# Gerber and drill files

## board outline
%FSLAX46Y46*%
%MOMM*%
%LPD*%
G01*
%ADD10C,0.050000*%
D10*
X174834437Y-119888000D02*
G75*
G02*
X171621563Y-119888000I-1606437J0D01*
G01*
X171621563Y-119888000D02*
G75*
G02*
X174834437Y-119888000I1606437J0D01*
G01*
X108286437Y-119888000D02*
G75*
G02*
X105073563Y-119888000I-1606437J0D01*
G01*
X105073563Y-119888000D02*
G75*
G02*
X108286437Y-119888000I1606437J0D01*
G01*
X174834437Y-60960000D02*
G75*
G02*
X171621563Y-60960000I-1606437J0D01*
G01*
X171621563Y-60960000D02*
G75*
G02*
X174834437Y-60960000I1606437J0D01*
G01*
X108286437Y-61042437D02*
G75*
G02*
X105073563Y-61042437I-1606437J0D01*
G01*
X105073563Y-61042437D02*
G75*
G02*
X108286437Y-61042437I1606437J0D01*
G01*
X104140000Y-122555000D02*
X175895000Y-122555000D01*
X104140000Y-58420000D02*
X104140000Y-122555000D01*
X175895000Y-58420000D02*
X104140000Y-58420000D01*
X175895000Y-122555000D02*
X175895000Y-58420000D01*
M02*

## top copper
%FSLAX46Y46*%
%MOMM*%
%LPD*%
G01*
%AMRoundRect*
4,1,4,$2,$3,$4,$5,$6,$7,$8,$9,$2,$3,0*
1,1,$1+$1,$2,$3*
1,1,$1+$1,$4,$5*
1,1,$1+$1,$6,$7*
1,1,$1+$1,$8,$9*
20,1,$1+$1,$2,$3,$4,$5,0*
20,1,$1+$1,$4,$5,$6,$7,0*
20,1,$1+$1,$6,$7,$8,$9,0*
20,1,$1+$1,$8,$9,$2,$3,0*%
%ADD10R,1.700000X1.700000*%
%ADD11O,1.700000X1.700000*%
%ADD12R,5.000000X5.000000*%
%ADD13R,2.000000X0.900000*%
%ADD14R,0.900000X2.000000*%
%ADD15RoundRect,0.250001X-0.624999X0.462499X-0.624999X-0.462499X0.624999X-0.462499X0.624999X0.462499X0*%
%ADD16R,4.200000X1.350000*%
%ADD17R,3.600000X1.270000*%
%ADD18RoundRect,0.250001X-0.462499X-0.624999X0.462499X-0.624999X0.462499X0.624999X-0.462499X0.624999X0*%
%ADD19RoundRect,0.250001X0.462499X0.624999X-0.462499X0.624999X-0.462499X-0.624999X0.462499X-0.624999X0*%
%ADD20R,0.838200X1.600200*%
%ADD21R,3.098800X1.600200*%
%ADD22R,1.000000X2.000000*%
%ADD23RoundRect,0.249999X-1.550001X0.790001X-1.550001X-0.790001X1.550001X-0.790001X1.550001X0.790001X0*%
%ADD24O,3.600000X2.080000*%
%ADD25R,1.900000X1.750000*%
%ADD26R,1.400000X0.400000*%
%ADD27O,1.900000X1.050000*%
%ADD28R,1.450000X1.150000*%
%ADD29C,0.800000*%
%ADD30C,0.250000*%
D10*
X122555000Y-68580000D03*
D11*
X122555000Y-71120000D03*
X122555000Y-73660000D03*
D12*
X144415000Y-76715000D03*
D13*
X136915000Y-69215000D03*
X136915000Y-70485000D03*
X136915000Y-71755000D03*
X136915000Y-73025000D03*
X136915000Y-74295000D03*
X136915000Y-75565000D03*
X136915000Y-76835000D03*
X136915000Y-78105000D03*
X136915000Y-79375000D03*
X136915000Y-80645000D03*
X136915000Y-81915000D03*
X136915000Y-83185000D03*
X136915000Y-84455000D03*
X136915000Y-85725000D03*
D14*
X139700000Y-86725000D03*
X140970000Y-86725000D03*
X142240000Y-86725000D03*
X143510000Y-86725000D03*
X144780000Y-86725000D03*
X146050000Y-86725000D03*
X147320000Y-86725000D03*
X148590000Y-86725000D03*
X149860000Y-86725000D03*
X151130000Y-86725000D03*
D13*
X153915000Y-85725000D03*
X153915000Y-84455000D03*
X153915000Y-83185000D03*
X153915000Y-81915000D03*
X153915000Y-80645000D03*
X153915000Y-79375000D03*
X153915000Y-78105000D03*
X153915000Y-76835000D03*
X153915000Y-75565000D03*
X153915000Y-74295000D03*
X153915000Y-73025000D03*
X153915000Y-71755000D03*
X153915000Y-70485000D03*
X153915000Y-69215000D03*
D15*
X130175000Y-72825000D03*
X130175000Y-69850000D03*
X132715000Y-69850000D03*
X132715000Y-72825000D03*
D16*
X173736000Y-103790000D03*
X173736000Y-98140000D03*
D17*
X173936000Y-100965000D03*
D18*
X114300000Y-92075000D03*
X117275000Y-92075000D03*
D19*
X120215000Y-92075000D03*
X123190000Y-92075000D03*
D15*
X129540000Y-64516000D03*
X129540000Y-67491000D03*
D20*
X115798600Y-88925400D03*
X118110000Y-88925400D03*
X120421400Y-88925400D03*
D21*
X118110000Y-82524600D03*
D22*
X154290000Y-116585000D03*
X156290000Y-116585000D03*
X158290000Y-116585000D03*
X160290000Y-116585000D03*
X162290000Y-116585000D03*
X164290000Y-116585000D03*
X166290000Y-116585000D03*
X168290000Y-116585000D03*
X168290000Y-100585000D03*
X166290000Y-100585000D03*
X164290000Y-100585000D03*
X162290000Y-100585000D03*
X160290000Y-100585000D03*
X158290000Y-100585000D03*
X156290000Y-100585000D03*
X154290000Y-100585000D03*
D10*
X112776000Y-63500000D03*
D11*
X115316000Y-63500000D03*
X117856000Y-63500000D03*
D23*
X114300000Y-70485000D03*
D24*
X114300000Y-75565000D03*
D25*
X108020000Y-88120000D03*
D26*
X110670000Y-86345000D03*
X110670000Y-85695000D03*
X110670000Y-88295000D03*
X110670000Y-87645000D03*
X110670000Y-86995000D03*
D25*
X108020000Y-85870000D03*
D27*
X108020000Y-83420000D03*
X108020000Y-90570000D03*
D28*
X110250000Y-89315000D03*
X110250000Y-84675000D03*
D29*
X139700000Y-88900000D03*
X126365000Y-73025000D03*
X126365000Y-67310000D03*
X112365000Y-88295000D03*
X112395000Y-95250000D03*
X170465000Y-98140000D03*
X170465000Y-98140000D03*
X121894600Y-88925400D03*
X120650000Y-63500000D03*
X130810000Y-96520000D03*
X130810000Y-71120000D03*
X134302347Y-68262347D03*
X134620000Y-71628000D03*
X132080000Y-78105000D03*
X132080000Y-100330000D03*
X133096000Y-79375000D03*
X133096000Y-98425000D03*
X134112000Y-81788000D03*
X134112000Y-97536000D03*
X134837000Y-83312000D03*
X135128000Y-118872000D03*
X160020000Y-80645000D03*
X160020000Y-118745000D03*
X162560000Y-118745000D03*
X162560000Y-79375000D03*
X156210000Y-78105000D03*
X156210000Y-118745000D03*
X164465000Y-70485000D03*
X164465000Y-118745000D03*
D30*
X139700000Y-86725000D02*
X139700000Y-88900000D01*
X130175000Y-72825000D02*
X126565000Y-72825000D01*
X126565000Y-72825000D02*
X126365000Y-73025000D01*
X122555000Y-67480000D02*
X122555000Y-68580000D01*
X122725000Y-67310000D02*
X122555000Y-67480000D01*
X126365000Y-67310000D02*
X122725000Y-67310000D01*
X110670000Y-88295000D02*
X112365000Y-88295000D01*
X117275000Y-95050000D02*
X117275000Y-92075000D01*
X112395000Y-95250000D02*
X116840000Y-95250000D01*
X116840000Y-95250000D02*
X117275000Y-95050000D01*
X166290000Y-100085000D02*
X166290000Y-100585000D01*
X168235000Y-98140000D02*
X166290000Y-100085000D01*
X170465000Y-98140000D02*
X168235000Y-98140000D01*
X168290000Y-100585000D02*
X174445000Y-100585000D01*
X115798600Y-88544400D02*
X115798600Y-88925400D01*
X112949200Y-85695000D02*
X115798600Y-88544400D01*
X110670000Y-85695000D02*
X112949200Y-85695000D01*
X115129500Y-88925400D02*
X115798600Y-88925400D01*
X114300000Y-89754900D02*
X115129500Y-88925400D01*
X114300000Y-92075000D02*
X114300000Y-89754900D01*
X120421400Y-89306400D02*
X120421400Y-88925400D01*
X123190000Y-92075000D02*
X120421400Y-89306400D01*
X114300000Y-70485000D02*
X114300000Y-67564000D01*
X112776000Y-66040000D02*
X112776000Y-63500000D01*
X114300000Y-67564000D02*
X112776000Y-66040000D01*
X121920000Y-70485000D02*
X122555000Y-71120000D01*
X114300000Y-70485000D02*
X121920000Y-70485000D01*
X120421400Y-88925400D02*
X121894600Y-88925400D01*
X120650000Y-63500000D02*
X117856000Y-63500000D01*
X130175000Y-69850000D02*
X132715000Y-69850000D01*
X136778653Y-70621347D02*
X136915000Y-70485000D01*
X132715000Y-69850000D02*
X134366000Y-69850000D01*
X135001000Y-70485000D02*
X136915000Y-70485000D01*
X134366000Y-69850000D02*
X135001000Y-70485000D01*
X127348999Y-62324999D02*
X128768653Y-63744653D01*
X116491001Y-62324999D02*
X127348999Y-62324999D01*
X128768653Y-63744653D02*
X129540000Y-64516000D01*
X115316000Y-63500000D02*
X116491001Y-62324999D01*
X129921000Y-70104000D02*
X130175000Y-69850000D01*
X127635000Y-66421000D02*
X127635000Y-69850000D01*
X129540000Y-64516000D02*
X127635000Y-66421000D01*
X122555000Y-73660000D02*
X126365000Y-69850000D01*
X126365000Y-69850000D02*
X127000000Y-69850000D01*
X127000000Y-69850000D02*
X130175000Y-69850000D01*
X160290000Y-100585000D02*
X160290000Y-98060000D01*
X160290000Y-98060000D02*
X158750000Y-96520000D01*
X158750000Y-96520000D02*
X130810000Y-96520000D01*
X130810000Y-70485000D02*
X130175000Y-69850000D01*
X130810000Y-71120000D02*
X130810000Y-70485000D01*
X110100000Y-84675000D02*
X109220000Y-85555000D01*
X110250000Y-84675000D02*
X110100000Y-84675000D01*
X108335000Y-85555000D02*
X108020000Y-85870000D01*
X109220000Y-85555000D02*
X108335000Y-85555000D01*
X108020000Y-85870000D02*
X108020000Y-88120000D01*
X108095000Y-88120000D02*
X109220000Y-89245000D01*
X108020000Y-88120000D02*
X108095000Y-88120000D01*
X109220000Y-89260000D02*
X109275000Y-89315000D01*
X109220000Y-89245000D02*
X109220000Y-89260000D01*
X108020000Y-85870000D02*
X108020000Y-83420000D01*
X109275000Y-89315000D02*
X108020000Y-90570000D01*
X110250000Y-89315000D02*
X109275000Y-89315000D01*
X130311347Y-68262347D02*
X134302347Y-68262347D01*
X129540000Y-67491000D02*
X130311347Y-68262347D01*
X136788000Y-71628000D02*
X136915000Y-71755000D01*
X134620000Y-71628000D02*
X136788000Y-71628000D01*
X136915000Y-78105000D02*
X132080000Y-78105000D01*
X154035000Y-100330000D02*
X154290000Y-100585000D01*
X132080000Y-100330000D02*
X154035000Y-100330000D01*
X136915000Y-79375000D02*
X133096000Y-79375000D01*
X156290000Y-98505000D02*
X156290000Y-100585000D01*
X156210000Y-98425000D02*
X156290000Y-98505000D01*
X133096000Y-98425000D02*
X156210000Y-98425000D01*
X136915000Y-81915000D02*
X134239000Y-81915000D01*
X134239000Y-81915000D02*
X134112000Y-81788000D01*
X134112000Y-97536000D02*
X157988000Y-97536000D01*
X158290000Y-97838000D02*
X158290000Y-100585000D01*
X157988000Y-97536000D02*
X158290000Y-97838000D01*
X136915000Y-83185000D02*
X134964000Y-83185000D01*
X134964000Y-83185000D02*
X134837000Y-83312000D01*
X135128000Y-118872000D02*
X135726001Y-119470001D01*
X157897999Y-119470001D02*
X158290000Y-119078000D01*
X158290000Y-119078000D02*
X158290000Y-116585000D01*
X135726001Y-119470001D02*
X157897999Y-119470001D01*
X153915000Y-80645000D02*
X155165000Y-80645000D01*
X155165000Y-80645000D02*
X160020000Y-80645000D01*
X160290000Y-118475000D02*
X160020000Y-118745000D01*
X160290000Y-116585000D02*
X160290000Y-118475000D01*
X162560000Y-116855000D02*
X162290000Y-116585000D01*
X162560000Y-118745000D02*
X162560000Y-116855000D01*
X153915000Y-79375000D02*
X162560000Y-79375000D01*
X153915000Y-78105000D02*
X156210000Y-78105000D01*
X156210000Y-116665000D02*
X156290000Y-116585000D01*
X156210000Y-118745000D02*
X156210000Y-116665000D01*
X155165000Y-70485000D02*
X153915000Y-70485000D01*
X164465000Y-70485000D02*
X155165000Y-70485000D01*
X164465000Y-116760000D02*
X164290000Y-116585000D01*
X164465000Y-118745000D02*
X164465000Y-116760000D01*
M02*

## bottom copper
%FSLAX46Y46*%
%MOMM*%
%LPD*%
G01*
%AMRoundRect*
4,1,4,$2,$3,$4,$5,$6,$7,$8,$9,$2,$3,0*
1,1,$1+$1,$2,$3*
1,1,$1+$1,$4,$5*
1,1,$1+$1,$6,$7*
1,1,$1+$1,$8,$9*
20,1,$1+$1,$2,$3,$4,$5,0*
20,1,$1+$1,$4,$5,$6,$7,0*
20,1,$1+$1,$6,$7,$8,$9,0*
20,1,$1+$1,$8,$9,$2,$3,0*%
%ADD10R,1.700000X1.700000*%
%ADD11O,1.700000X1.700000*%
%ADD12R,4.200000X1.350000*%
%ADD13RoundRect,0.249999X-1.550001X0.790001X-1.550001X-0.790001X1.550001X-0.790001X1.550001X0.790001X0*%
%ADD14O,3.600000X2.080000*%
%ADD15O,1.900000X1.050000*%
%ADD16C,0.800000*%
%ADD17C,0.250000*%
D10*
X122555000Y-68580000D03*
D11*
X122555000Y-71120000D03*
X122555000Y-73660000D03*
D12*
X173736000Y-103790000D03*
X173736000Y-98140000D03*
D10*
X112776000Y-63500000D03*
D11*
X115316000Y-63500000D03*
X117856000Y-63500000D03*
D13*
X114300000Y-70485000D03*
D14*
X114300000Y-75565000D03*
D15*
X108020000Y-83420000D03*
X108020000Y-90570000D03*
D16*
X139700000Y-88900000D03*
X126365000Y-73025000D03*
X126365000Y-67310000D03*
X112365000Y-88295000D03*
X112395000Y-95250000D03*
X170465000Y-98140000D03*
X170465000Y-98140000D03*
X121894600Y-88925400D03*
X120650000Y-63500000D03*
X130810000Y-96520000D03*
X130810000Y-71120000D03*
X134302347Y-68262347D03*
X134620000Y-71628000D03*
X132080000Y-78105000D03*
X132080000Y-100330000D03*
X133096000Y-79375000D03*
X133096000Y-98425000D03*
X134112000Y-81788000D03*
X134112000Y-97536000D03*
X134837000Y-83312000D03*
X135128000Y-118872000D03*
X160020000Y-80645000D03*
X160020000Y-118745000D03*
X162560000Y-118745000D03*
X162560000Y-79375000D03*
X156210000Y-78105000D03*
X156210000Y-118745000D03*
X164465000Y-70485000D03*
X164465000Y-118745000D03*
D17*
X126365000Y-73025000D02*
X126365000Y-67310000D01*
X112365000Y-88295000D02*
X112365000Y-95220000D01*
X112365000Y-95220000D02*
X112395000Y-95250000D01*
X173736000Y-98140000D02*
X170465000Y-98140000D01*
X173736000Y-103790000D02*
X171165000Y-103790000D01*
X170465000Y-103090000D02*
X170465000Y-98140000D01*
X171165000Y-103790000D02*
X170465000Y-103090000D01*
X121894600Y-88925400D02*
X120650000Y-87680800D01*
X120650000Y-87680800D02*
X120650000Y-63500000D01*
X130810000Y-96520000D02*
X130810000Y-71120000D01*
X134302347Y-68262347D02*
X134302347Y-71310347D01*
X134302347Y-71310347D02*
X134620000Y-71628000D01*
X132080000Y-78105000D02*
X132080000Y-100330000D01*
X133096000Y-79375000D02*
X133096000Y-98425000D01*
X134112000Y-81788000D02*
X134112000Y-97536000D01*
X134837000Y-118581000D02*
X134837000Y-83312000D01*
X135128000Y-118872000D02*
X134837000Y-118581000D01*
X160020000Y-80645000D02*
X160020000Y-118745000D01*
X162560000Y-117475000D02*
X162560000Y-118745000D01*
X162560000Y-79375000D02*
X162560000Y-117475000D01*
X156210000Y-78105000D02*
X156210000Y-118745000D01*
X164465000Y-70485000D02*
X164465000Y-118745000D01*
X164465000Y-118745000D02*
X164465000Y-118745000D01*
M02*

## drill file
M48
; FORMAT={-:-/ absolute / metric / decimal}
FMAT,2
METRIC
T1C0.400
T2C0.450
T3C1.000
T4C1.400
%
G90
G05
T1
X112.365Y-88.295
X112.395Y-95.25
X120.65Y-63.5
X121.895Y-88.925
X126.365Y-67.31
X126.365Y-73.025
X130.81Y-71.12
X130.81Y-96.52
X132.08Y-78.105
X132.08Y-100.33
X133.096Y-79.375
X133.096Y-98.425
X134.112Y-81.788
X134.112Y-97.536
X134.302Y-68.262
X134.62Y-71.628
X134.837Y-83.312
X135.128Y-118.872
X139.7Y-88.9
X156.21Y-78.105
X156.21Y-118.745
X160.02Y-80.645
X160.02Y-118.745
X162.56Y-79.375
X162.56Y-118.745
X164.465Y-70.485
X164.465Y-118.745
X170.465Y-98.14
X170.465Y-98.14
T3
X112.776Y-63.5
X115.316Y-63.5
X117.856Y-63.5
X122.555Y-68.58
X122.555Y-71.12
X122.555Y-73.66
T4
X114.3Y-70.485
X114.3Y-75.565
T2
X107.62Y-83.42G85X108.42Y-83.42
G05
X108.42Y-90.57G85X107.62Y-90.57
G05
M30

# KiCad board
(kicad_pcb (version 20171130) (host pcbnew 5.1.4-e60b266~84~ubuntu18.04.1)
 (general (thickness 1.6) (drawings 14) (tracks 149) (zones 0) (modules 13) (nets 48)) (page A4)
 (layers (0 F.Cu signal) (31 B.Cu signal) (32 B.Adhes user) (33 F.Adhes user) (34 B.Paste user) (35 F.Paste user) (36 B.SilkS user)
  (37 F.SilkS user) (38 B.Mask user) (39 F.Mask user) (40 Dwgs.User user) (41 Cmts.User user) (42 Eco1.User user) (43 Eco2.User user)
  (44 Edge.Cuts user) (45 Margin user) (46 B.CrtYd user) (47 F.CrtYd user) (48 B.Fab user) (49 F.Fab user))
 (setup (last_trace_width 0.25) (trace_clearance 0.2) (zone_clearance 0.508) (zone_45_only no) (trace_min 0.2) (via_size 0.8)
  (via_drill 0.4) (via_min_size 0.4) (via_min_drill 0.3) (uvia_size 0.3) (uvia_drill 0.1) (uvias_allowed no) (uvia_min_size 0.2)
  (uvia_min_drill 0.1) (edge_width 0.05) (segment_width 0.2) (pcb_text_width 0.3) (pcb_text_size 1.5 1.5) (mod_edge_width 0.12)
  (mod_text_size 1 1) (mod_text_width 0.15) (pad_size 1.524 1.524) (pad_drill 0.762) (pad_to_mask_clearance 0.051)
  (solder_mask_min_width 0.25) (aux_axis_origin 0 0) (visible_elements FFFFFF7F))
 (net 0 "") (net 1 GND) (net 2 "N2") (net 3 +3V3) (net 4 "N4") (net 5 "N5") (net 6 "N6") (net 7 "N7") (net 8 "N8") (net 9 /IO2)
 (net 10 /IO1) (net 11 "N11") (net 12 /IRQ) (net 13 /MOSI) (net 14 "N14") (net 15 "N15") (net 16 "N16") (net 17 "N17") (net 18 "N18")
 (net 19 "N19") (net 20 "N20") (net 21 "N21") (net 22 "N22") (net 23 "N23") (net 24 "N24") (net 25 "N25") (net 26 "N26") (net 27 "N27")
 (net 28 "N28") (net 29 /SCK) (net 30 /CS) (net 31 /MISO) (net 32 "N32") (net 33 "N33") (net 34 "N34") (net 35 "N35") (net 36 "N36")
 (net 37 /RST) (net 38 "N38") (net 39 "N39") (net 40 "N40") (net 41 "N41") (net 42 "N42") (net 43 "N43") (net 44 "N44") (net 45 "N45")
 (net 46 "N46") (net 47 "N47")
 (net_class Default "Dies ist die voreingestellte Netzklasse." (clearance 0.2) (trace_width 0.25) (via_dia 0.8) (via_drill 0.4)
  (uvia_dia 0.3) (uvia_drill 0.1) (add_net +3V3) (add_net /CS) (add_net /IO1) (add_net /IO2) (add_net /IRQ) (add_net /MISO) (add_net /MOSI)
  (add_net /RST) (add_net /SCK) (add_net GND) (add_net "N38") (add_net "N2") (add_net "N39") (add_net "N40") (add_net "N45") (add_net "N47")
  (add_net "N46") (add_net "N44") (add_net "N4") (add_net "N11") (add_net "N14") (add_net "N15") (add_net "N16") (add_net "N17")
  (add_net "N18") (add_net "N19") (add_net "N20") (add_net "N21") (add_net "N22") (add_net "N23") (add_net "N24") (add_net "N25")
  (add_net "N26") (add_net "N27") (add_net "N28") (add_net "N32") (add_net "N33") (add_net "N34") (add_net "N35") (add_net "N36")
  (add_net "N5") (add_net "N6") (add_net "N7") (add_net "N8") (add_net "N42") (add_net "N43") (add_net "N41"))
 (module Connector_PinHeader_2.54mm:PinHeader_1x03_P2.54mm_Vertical (layer F.Cu) (at 122.555 68.58)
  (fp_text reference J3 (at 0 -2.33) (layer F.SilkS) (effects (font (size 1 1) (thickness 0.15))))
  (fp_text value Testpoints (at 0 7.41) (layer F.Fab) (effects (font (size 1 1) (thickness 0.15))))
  (pad 1 thru_hole rect (at 0 0) (size 1.7 1.7) (drill 1) (layers *.Cu *.Mask) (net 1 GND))
  (pad 2 thru_hole oval (at 0 2.54) (size 1.7 1.7) (drill 1) (layers *.Cu *.Mask) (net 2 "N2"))
  (pad 3 thru_hole oval (at 0 5.08) (size 1.7 1.7) (drill 1) (layers *.Cu *.Mask) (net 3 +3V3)))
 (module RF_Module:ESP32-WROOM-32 (layer F.Cu) (at 145.415 77.47)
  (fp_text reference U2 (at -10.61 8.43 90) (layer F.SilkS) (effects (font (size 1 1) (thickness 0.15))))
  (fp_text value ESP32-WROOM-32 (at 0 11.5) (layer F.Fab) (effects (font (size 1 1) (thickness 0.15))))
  (pad 39 smd rect (at -1 -0.755) (size 5 5) (layers F.Cu F.Paste F.Mask))
  (pad 1 smd rect (at -8.5 -8.255) (size 2 0.9) (layers F.Cu F.Paste F.Mask) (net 1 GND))
  (pad 2 smd rect (at -8.5 -6.985) (size 2 0.9) (layers F.Cu F.Paste F.Mask) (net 3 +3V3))
  (pad 3 smd rect (at -8.5 -5.715) (size 2 0.9) (layers F.Cu F.Paste F.Mask) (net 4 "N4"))
  (pad 4 smd rect (at -8.5 -4.445) (size 2 0.9) (layers F.Cu F.Paste F.Mask) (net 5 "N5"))
  (pad 5 smd rect (at -8.5 -3.175) (size 2 0.9) (layers F.Cu F.Paste F.Mask) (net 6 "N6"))
  (pad 6 smd rect (at -8.5 -1.905) (size 2 0.9) (layers F.Cu F.Paste F.Mask) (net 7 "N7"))
  (pad 7 smd rect (at -8.5 -0.635) (size 2 0.9) (layers F.Cu F.Paste F.Mask) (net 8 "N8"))
  (pad 8 smd rect (at -8.5 0.635) (size 2 0.9) (layers F.Cu F.Paste F.Mask) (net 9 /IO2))
  (pad 9 smd rect (at -8.5 1.905) (size 2 0.9) (layers F.Cu F.Paste F.Mask) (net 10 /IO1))
  (pad 10 smd rect (at -8.5 3.175) (size 2 0.9) (layers F.Cu F.Paste F.Mask) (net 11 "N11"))
  (pad 11 smd rect (at -8.5 4.445) (size 2 0.9) (layers F.Cu F.Paste F.Mask) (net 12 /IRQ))
  (pad 12 smd rect (at -8.5 5.715) (size 2 0.9) (layers F.Cu F.Paste F.Mask) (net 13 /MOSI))
  (pad 13 smd rect (at -8.5 6.985) (size 2 0.9) (layers F.Cu F.Paste F.Mask) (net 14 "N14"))
  (pad 14 smd rect (at -8.5 8.255) (size 2 0.9) (layers F.Cu F.Paste F.Mask) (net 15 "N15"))
  (pad 15 smd rect (at -5.715 9.255 90) (size 2 0.9) (layers F.Cu F.Paste F.Mask) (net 1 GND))
  (pad 16 smd rect (at -4.445 9.255 90) (size 2 0.9) (layers F.Cu F.Paste F.Mask) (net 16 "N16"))
  (pad 17 smd rect (at -3.175 9.255 90) (size 2 0.9) (layers F.Cu F.Paste F.Mask) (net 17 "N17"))
  (pad 18 smd rect (at -1.905 9.255 90) (size 2 0.9) (layers F.Cu F.Paste F.Mask) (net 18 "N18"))
  (pad 19 smd rect (at -0.635 9.255 90) (size 2 0.9) (layers F.Cu F.Paste F.Mask) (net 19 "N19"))
  (pad 20 smd rect (at 0.635 9.255 90) (size 2 0.9) (layers F.Cu F.Paste F.Mask) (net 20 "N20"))
  (pad 21 smd rect (at 1.905 9.255 90) (size 2 0.9) (layers F.Cu F.Paste F.Mask) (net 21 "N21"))
  (pad 22 smd rect (at 3.175 9.255 90) (size 2 0.9) (layers F.Cu F.Paste F.Mask) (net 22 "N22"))
  (pad 23 smd rect (at 4.445 9.255 90) (size 2 0.9) (layers F.Cu F.Paste F.Mask) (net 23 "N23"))
  (pad 24 smd rect (at 5.715 9.255 90) (size 2 0.9) (layers F.Cu F.Paste F.Mask) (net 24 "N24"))
  (pad 25 smd rect (at 8.5 8.255) (size 2 0.9) (layers F.Cu F.Paste F.Mask) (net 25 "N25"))
  (pad 26 smd rect (at 8.5 6.985) (size 2 0.9) (layers F.Cu F.Paste F.Mask) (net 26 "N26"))
  (pad 27 smd rect (at 8.5 5.715) (size 2 0.9) (layers F.Cu F.Paste F.Mask) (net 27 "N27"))
  (pad 28 smd rect (at 8.5 4.445) (size 2 0.9) (layers F.Cu F.Paste F.Mask) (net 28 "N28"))
  (pad 29 smd rect (at 8.5 3.175) (size 2 0.9) (layers F.Cu F.Paste F.Mask) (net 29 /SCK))
  (pad 30 smd rect (at 8.5 1.905) (size 2 0.9) (layers F.Cu F.Paste F.Mask) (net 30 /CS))
  (pad 31 smd rect (at 8.5 0.635) (size 2 0.9) (layers F.Cu F.Paste F.Mask) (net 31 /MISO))
  (pad 32 smd rect (at 8.5 -0.635) (size 2 0.9) (layers F.Cu F.Paste F.Mask) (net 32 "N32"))
  (pad 33 smd rect (at 8.5 -1.905) (size 2 0.9) (layers F.Cu F.Paste F.Mask) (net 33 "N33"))
  (pad 34 smd rect (at 8.5 -3.175) (size 2 0.9) (layers F.Cu F.Paste F.Mask) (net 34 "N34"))
  (pad 35 smd rect (at 8.5 -4.445) (size 2 0.9) (layers F.Cu F.Paste F.Mask) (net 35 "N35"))
  (pad 36 smd rect (at 8.5 -5.715) (size 2 0.9) (layers F.Cu F.Paste F.Mask) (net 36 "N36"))
  (pad 37 smd rect (at 8.5 -6.985) (size 2 0.9) (layers F.Cu F.Paste F.Mask) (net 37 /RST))
  (pad 38 smd rect (at 8.5 -8.255) (size 2 0.9) (layers F.Cu F.Paste F.Mask) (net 1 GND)))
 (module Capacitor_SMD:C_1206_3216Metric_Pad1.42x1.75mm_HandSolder (layer F.Cu) (at 130.175 71.3375 270)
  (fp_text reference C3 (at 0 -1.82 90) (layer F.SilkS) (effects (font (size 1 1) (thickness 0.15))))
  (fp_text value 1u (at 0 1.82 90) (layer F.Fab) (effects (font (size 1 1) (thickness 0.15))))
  (pad 2 smd roundrect (at 1.4875 0 270) (size 1.425 1.75) (layers F.Cu F.Paste F.Mask) (roundrect_rratio 0.175439) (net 1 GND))
  (pad 1 smd roundrect (at -1.4875 0 270) (size 1.425 1.75) (layers F.Cu F.Paste F.Mask) (roundrect_rratio 0.175439) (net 3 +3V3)))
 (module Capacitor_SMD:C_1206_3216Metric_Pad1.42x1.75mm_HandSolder (layer F.Cu) (at 132.715 71.3375 270)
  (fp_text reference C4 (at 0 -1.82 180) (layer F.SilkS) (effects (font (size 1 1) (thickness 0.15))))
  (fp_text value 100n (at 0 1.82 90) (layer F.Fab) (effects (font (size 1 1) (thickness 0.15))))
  (pad 1 smd roundrect (at -1.4875 0 270) (size 1.425 1.75) (layers F.Cu F.Paste F.Mask) (roundrect_rratio 0.175439) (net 3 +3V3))
  (pad 2 smd roundrect (at 1.4875 0 270) (size 1.425 1.75) (layers F.Cu F.Paste F.Mask) (roundrect_rratio 0.175439) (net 1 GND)))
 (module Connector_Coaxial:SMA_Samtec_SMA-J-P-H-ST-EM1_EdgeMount (layer F.Cu) (at 173.736 100.965)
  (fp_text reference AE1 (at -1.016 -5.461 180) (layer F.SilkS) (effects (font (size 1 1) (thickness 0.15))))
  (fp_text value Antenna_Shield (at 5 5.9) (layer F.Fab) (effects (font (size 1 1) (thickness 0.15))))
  (pad 2 smd rect (at 0 2.825 90) (size 1.35 4.2) (layers B.Cu B.Paste B.Mask) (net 1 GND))
  (pad 2 smd rect (at 0 -2.825 90) (size 1.35 4.2) (layers B.Cu B.Paste B.Mask) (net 1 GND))
  (pad 2 smd rect (at 0 2.825 90) (size 1.35 4.2) (layers F.Cu F.Paste F.Mask) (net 1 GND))
  (pad 2 smd rect (at 0 -2.825 90) (size 1.35 4.2) (layers F.Cu F.Paste F.Mask) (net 1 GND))
  (pad 1 smd rect (at 0.2 0 90) (size 1.27 3.6) (layers F.Cu F.Paste F.Mask) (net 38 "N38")))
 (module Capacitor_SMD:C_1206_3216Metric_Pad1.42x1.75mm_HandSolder (layer F.Cu) (at 115.7875 92.075)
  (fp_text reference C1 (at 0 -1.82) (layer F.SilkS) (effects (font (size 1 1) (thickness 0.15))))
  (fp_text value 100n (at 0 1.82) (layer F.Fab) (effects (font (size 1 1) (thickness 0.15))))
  (pad 1 smd roundrect (at -1.4875 0) (size 1.425 1.75) (layers F.Cu F.Paste F.Mask) (roundrect_rratio 0.175439) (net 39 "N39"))
  (pad 2 smd roundrect (at 1.4875 0) (size 1.425 1.75) (layers F.Cu F.Paste F.Mask) (roundrect_rratio 0.175439) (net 1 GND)))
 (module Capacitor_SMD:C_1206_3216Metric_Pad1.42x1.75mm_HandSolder (layer F.Cu) (at 121.7025 92.075 180)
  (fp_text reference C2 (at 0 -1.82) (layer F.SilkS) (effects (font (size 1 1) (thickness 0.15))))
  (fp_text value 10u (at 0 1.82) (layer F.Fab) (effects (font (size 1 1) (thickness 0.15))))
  (pad 2 smd roundrect (at 1.4875 0 180) (size 1.425 1.75) (layers F.Cu F.Paste F.Mask) (roundrect_rratio 0.175439) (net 1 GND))
  (pad 1 smd roundrect (at -1.4875 0 180) (size 1.425 1.75) (layers F.Cu F.Paste F.Mask) (roundrect_rratio 0.175439) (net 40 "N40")))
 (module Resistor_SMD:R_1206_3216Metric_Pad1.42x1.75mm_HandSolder (layer F.Cu) (at 129.54 66.0035 270)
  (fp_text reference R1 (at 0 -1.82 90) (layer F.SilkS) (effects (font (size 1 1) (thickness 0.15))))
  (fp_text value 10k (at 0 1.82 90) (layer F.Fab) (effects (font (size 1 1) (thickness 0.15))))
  (pad 1 smd roundrect (at -1.4875 0 270) (size 1.425 1.75) (layers F.Cu F.Paste F.Mask) (roundrect_rratio 0.175439) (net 3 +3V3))
  (pad 2 smd roundrect (at 1.4875 0 270) (size 1.425 1.75) (layers F.Cu F.Paste F.Mask) (roundrect_rratio 0.175439) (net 4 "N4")))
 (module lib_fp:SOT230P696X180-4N (layer F.Cu) (at 118.11 85.725 90)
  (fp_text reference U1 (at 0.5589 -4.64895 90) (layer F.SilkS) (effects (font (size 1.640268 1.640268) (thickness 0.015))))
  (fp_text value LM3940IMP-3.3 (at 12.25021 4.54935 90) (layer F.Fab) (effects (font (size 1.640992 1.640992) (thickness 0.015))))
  (pad 1 smd rect (at -3.2004 -2.3114 90) (size 1.6002 0.8382) (layers F.Cu F.Paste F.Mask) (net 39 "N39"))
  (pad 2 smd rect (at -3.2004 0 90) (size 1.6002 0.8382) (layers F.Cu F.Paste F.Mask) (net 1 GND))
  (pad 3 smd rect (at -3.2004 2.3114 90) (size 1.6002 0.8382) (layers F.Cu F.Paste F.Mask) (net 40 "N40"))
  (pad 4 smd rect (at 3.2004 0 90) (size 1.6002 3.0988) (layers F.Cu F.Paste F.Mask) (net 1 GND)))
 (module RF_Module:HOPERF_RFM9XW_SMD (layer F.Cu) (at 161.29 108.585 90)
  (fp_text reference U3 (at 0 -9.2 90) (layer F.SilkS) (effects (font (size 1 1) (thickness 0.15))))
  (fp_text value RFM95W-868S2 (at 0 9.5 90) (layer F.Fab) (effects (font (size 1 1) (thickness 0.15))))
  (pad 1 smd rect (at -8 -7 90) (size 2 1) (layers F.Cu F.Paste F.Mask) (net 1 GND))
  (pad 2 smd rect (at -8 -5 90) (size 2 1) (layers F.Cu F.Paste F.Mask) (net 31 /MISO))
  (pad 3 smd rect (at -8 -3 90) (size 2 1) (layers F.Cu F.Paste F.Mask) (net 13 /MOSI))
  (pad 4 smd rect (at -8 -1 90) (size 2 1) (layers F.Cu F.Paste F.Mask) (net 29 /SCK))
  (pad 5 smd rect (at -8 1 90) (size 2 1) (layers F.Cu F.Paste F.Mask) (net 30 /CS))
  (pad 6 smd rect (at -8 3 90) (size 2 1) (layers F.Cu F.Paste F.Mask) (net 37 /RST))
  (pad 7 smd rect (at -8 5 90) (size 2 1) (layers F.Cu F.Paste F.Mask) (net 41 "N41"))
  (pad 8 smd rect (at -8 7 90) (size 2 1) (layers F.Cu F.Paste F.Mask) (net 1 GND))
  (pad 9 smd rect (at 8 7 90) (size 2 1) (layers F.Cu F.Paste F.Mask) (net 38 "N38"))
  (pad 10 smd rect (at 8 5 90) (size 2 1) (layers F.Cu F.Paste F.Mask) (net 1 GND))
  (pad 11 smd rect (at 8 3 90) (size 2 1) (layers F.Cu F.Paste F.Mask) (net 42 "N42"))
  (pad 12 smd rect (at 8 1 90) (size 2 1) (layers F.Cu F.Paste F.Mask) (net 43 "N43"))
  (pad 13 smd rect (at 8 -1 90) (size 2 1) (layers F.Cu F.Paste F.Mask) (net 3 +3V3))
  (pad 14 smd rect (at 8 -3 90) (size 2 1) (layers F.Cu F.Paste F.Mask) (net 12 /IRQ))
  (pad 15 smd rect (at 8 -5 90) (size 2 1) (layers F.Cu F.Paste F.Mask) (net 10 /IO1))
  (pad 16 smd rect (at 8 -7 90) (size 2 1) (layers F.Cu F.Paste F.Mask) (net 9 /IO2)))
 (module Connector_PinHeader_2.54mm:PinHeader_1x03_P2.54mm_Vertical (layer F.Cu) (at 112.776 63.5 90)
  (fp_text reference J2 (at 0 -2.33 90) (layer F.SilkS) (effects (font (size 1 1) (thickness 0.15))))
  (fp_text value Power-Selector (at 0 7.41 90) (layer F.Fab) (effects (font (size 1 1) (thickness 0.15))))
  (pad 1 thru_hole rect (at 0 0 90) (size 1.7 1.7) (drill 1) (layers *.Cu *.Mask) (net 2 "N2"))
  (pad 2 thru_hole oval (at 0 2.54 90) (size 1.7 1.7) (drill 1) (layers *.Cu *.Mask) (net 3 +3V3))
  (pad 3 thru_hole oval (at 0 5.08 90) (size 1.7 1.7) (drill 1) (layers *.Cu *.Mask) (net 40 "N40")))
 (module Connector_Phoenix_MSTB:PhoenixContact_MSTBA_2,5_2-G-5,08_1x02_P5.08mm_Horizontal (layer F.Cu) (at 114.3 70.485 270)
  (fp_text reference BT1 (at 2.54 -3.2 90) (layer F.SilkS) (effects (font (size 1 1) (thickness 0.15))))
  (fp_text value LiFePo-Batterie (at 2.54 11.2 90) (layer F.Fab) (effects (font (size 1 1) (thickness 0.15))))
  (pad 1 thru_hole roundrect (at 0 0 270) (size 2.08 3.6) (drill 1.4) (layers *.Cu *.Mask) (roundrect_rratio 0.120192) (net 2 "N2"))
  (pad 2 thru_hole oval (at 5.08 0 270) (size 2.08 3.6) (drill 1.4) (layers *.Cu *.Mask) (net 1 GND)))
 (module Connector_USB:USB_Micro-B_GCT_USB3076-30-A (layer F.Cu) (at 109.22 86.995 270)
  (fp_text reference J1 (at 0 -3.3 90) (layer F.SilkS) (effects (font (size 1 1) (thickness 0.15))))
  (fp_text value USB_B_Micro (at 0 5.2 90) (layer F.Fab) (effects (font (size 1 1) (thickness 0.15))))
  (pad 6 smd rect (at 1.125 1.2 270) (size 1.75 1.9) (layers F.Cu F.Paste F.Mask) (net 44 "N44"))
  (pad 2 smd rect (at -0.65 -1.45 270) (size 0.4 1.4) (layers F.Cu F.Paste F.Mask) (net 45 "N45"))
  (pad 1 smd rect (at -1.3 -1.45 270) (size 0.4 1.4) (layers F.Cu F.Paste F.Mask) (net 39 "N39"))
  (pad 5 smd rect (at 1.3 -1.45 270) (size 0.4 1.4) (layers F.Cu F.Paste F.Mask) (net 1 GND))
  (pad 4 smd rect (at 0.65 -1.45 270) (size 0.4 1.4) (layers F.Cu F.Paste F.Mask) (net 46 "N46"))
  (pad 3 smd rect (at 0 -1.45 270) (size 0.4 1.4) (layers F.Cu F.Paste F.Mask) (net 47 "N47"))
  (pad 6 smd rect (at -1.125 1.2 270) (size 1.75 1.9) (layers F.Cu F.Paste F.Mask) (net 44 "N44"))
  (pad 6 thru_hole oval (at -3.575 1.2 90) (size 1.05 1.9) (drill oval 0.45 1.25) (layers *.Cu *.Mask) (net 44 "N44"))
  (pad 6 thru_hole oval (at 3.575 1.2 270) (size 1.05 1.9) (drill oval 0.45 1.25) (layers *.Cu *.Mask) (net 44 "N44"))
  (pad 6 smd rect (at 2.32 -1.03 270) (size 1.15 1.45) (layers F.Cu F.Paste F.Mask) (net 44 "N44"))
  (pad 6 smd rect (at -2.32 -1.03 270) (size 1.15 1.45) (layers F.Cu F.Paste F.Mask) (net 44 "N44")))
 (gr_circle (center 173.228 119.888) (end 173.736 121.412) (layer Edge.Cuts) (width 0.05))
 (gr_circle (center 106.68 119.888) (end 107.188 121.412) (layer Edge.Cuts) (width 0.05))
 (gr_circle (center 173.228 60.96) (end 173.736 62.484) (layer Edge.Cuts) (width 0.05))
 (gr_circle (center 106.68 61.042437) (end 107.188 62.566437) (layer Edge.Cuts) (width 0.05))
 (gr_line (start 104.14 122.555) (end 175.895 122.555) (layer Edge.Cuts) (width 0.05))
 (gr_line (start 104.14 58.42) (end 104.14 122.555) (layer Edge.Cuts) (width 0.05))
 (gr_line (start 175.895 58.42) (end 104.14 58.42) (layer Edge.Cuts) (width 0.05))
 (gr_line (start 175.895 122.555) (end 175.895 58.42) (layer Edge.Cuts) (width 0.05))
 (segment (start 139.7 86.725) (end 139.7 88.9) (width 0.25) (layer F.Cu) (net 1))
 (via (at 139.7 88.9) (size 0.8) (drill 0.4) (layers F.Cu B.Cu) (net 1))
 (via (at 126.365 73.025) (size 0.8) (drill 0.4) (layers F.Cu B.Cu) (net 1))
 (segment (start 130.175 72.825) (end 126.565 72.825) (width 0.25) (layer F.Cu) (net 1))
 (segment (start 126.565 72.825) (end 126.365 73.025) (width 0.25) (layer F.Cu) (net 1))
 (segment (start 126.365 73.025) (end 126.365 67.31) (width 0.25) (layer B.Cu) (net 1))
 (via (at 126.365 67.31) (size 0.8) (drill 0.4) (layers F.Cu B.Cu) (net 1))
 (segment (start 122.555 67.48) (end 122.555 68.58) (width 0.25) (layer F.Cu) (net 1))
 (segment (start 122.725 67.31) (end 122.555 67.48) (width 0.25) (layer F.Cu) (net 1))
 (segment (start 126.365 67.31) (end 122.725 67.31) (width 0.25) (layer F.Cu) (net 1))
 (segment (start 110.67 88.295) (end 112.365 88.295) (width 0.25) (layer F.Cu) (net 1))
 (via (at 112.365 88.295) (size 0.8) (drill 0.4) (layers F.Cu B.Cu) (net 1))
 (segment (start 112.365 88.295) (end 112.365 95.22) (width 0.25) (layer B.Cu) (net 1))
 (via (at 112.395 95.25) (size 0.8) (drill 0.4) (layers F.Cu B.Cu) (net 1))
 (segment (start 112.365 95.22) (end 112.395 95.25) (width 0.25) (layer B.Cu) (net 1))
 (segment (start 117.275 95.05) (end 117.275 92.075) (width 0.25) (layer F.Cu) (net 1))
 (segment (start 112.395 95.25) (end 116.84 95.25) (width 0.25) (layer F.Cu) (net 1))
 (segment (start 116.84 95.25) (end 117.275 95.05) (width 0.25) (layer F.Cu) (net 1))
 (segment (start 173.736 98.14) (end 170.465 98.14) (width 0.25) (layer B.Cu) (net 1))
 (via (at 170.465 98.14) (size 0.8) (drill 0.4) (layers F.Cu B.Cu) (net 1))
 (via (at 170.465 98.14) (size 0.8) (drill 0.4) (layers F.Cu B.Cu) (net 1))
 (segment (start 166.29 100.085) (end 166.29 100.585) (width 0.25) (layer F.Cu) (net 1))
 (segment (start 168.235 98.14) (end 166.29 100.085) (width 0.25) (layer F.Cu) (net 1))
 (segment (start 170.465 98.14) (end 168.235 98.14) (width 0.25) (layer F.Cu) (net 1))
 (segment (start 173.736 103.79) (end 171.165 103.79) (width 0.25) (layer B.Cu) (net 1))
 (segment (start 170.465 103.09) (end 170.465 98.14) (width 0.25) (layer B.Cu) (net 1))
 (segment (start 171.165 103.79) (end 170.465 103.09) (width 0.25) (layer B.Cu) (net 1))
 (segment (start 168.29 100.585) (end 174.445 100.585) (width 0.25) (layer F.Cu) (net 38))
 (segment (start 115.7986 88.5444) (end 115.7986 88.9254) (width 0.25) (layer F.Cu) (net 39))
 (segment (start 112.9492 85.695) (end 115.7986 88.5444) (width 0.25) (layer F.Cu) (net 39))
 (segment (start 110.67 85.695) (end 112.9492 85.695) (width 0.25) (layer F.Cu) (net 39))
 (segment (start 115.1295 88.9254) (end 115.7986 88.9254) (width 0.25) (layer F.Cu) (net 39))
 (segment (start 114.3 89.7549) (end 115.1295 88.9254) (width 0.25) (layer F.Cu) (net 39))
 (segment (start 114.3 92.075) (end 114.3 89.7549) (width 0.25) (layer F.Cu) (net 39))
 (segment (start 120.4214 89.3064) (end 120.4214 88.9254) (width 0.25) (layer F.Cu) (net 40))
 (segment (start 123.19 92.075) (end 120.4214 89.3064) (width 0.25) (layer F.Cu) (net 40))
 (segment (start 114.3 70.485) (end 114.3 67.564) (width 0.25) (layer F.Cu) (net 2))
 (segment (start 112.776 66.04) (end 112.776 63.5) (width 0.25) (layer F.Cu) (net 2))
 (segment (start 114.3 67.564) (end 112.776 66.04) (width 0.25) (layer F.Cu) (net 2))
 (segment (start 121.92 70.485) (end 122.555 71.12) (width 0.25) (layer F.Cu) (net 2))
 (segment (start 114.3 70.485) (end 121.92 70.485) (width 0.25) (layer F.Cu) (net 2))
 (segment (start 120.4214 88.9254) (end 121.8946 88.9254) (width 0.25) (layer F.Cu) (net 40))
 (via (at 121.8946 88.9254) (size 0.8) (drill 0.4) (layers F.Cu B.Cu) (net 40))
 (segment (start 121.8946 88.9254) (end 120.65 87.6808) (width 0.25) (layer B.Cu) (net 40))
 (via (at 120.65 63.5) (size 0.8) (drill 0.4) (layers F.Cu B.Cu) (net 40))
 (segment (start 120.65 87.6808) (end 120.65 63.5) (width 0.25) (layer B.Cu) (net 40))
 (segment (start 120.65 63.5) (end 117.856 63.5) (width 0.25) (layer F.Cu) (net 40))
 (segment (start 130.175 69.85) (end 132.715 69.85) (width 0.25) (layer F.Cu) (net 3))
 (segment (start 136.778653 70.621347) (end 136.915 70.485) (width 0.25) (layer F.Cu) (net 3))
 (segment (start 132.715 69.85) (end 134.366 69.85) (width 0.25) (layer F.Cu) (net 3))
 (segment (start 135.001 70.485) (end 136.915 70.485) (width 0.25) (layer F.Cu) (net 3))
 (segment (start 134.366 69.85) (end 135.001 70.485) (width 0.25) (layer F.Cu) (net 3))
 (segment (start 127.348999 62.324999) (end 128.768653 63.744653) (width 0.25) (layer F.Cu) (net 3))
 (segment (start 116.491001 62.324999) (end 127.348999 62.324999) (width 0.25) (layer F.Cu) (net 3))
 (segment (start 128.768653 63.744653) (end 129.54 64.516) (width 0.25) (layer F.Cu) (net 3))
 (segment (start 115.316 63.5) (end 116.491001 62.324999) (width 0.25) (layer F.Cu) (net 3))
 (segment (start 129.921 70.104) (end 130.175 69.85) (width 0.25) (layer F.Cu) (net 3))
 (segment (start 127.635 66.421) (end 127.635 69.85) (width 0.25) (layer F.Cu) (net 3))
 (segment (start 129.54 64.516) (end 127.635 66.421) (width 0.25) (layer F.Cu) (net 3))
 (segment (start 122.555 73.66) (end 126.365 69.85) (width 0.25) (layer F.Cu) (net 3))
 (segment (start 126.365 69.85) (end 127 69.85) (width 0.25) (layer F.Cu) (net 3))
 (segment (start 127 69.85) (end 130.175 69.85) (width 0.25) (layer F.Cu) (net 3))
 (segment (start 160.29 100.585) (end 160.29 98.06) (width 0.25) (layer F.Cu) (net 3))
 (segment (start 160.29 98.06) (end 158.75 96.52) (width 0.25) (layer F.Cu) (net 3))
 (via (at 130.81 96.52) (size 0.8) (drill 0.4) (layers F.Cu B.Cu) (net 3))
 (segment (start 158.75 96.52) (end 130.81 96.52) (width 0.25) (layer F.Cu) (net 3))
 (segment (start 130.81 96.52) (end 130.81 71.12) (width 0.25) (layer B.Cu) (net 3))
 (via (at 130.81 71.12) (size 0.8) (drill 0.4) (layers F.Cu B.Cu) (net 3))
 (segment (start 130.81 70.485) (end 130.175 69.85) (width 0.25) (layer F.Cu) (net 3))
 (segment (start 130.81 71.12) (end 130.81 70.485) (width 0.25) (layer F.Cu) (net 3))
 (segment (start 110.1 84.675) (end 109.22 85.555) (width 0.25) (layer F.Cu) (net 44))
 (segment (start 110.25 84.675) (end 110.1 84.675) (width 0.25) (layer F.Cu) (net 44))
 (segment (start 108.335 85.555) (end 108.02 85.87) (width 0.25) (layer F.Cu) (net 44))
 (segment (start 109.22 85.555) (end 108.335 85.555) (width 0.25) (layer F.Cu) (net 44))
 (segment (start 108.02 85.87) (end 108.02 88.12) (width 0.25) (layer F.Cu) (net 44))
 (segment (start 108.095 88.12) (end 109.22 89.245) (width 0.25) (layer F.Cu) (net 44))
 (segment (start 108.02 88.12) (end 108.095 88.12) (width 0.25) (layer F.Cu) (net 44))
 (segment (start 109.22 89.26) (end 109.275 89.315) (width 0.25) (layer F.Cu) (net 44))
 (segment (start 109.22 89.245) (end 109.22 89.26) (width 0.25) (layer F.Cu) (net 44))
 (segment (start 108.02 85.87) (end 108.02 83.42) (width 0.25) (layer F.Cu) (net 44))
 (segment (start 109.275 89.315) (end 108.02 90.57) (width 0.25) (layer F.Cu) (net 44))
 (segment (start 110.25 89.315) (end 109.275 89.315) (width 0.25) (layer F.Cu) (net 44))
 (segment (start 130.311347 68.262347) (end 134.302347 68.262347) (width 0.25) (layer F.Cu) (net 4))
 (segment (start 129.54 67.491) (end 130.311347 68.262347) (width 0.25) (layer F.Cu) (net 4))
 (via (at 134.302347 68.262347) (size 0.8) (drill 0.4) (layers F.Cu B.Cu) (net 4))
 (via (at 134.62 71.628) (size 0.8) (drill 0.4) (layers F.Cu B.Cu) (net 4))
 (segment (start 134.302347 68.262347) (end 134.302347 71.310347) (width 0.25) (layer B.Cu) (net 4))
 (segment (start 134.302347 71.310347) (end 134.62 71.628) (width 0.25) (layer B.Cu) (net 4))
 (segment (start 136.788 71.628) (end 136.915 71.755) (width 0.25) (layer F.Cu) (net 4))
 (segment (start 134.62 71.628) (end 136.788 71.628) (width 0.25) (layer F.Cu) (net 4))
 (via (at 132.08 78.105) (size 0.8) (drill 0.4) (layers F.Cu B.Cu) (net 9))
 (segment (start 136.915 78.105) (end 132.08 78.105) (width 0.25) (layer F.Cu) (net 9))
 (via (at 132.08 100.33) (size 0.8) (drill 0.4) (layers F.Cu B.Cu) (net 9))
 (segment (start 132.08 78.105) (end 132.08 100.33) (width 0.25) (layer B.Cu) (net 9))
 (segment (start 154.035 100.33) (end 154.29 100.585) (width 0.25) (layer F.Cu) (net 9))
 (segment (start 132.08 100.33) (end 154.035 100.33) (width 0.25) (layer F.Cu) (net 9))
 (segment (start 136.915 79.375) (end 133.096 79.375) (width 0.25) (layer F.Cu) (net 10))
 (via (at 133.096 79.375) (size 0.8) (drill 0.4) (layers F.Cu B.Cu) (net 10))
 (segment (start 156.29 98.505) (end 156.29 100.585) (width 0.25) (layer F.Cu) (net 10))
 (segment (start 156.21 98.425) (end 156.29 98.505) (width 0.25) (layer F.Cu) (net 10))
 (segment (start 133.096 98.425) (end 156.21 98.425) (width 0.25) (layer F.Cu) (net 10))
 (via (at 133.096 98.425) (size 0.8) (drill 0.4) (layers F.Cu B.Cu) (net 10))
 (segment (start 133.096 79.375) (end 133.096 98.425) (width 0.25) (layer B.Cu) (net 10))
 (via (at 134.112 81.788) (size 0.8) (drill 0.4) (layers F.Cu B.Cu) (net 12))
 (segment (start 136.915 81.915) (end 134.239 81.915) (width 0.25) (layer F.Cu) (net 12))
 (segment (start 134.239 81.915) (end 134.112 81.788) (width 0.25) (layer F.Cu) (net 12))
 (segment (start 134.112 81.788) (end 134.112 97.536) (width 0.25) (layer B.Cu) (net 12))
 (via (at 134.112 97.536) (size 0.8) (drill 0.4) (layers F.Cu B.Cu) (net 12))
 (segment (start 134.112 97.536) (end 157.988 97.536) (width 0.25) (layer F.Cu) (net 12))
 (segment (start 158.29 97.838) (end 158.29 100.585) (width 0.25) (layer F.Cu) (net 12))
 (segment (start 157.988 97.536) (end 158.29 97.838) (width 0.25) (layer F.Cu) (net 12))
 (via (at 134.837 83.312) (size 0.8) (drill 0.4) (layers F.Cu B.Cu) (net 13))
 (segment (start 136.915 83.185) (end 134.964 83.185) (width 0.25) (layer F.Cu) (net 13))
 (segment (start 134.964 83.185) (end 134.837 83.312) (width 0.25) (layer F.Cu) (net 13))
 (segment (start 134.837 118.581) (end 134.837 83.312) (width 0.25) (layer B.Cu) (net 13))
 (segment (start 135.128 118.872) (end 135.726001 119.470001) (width 0.25) (layer F.Cu) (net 13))
 (segment (start 157.897999 119.470001) (end 158.29 119.078) (width 0.25) (layer F.Cu) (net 13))
 (segment (start 158.29 119.078) (end 158.29 116.585) (width 0.25) (layer F.Cu) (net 13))
 (segment (start 135.726001 119.470001) (end 157.897999 119.470001) (width 0.25) (layer F.Cu) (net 13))
 (via (at 135.128 118.872) (size 0.8) (drill 0.4) (layers F.Cu B.Cu) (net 13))
 (segment (start 135.128 118.872) (end 134.837 118.581) (width 0.25) (layer B.Cu) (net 13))
 (segment (start 153.915 80.645) (end 155.165 80.645) (width 0.25) (layer F.Cu) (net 29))
 (via (at 160.02 80.645) (size 0.8) (drill 0.4) (layers F.Cu B.Cu) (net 29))
 (segment (start 155.165 80.645) (end 160.02 80.645) (width 0.25) (layer F.Cu) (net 29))
 (segment (start 160.02 80.645) (end 160.02 118.745) (width 0.25) (layer B.Cu) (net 29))
 (via (at 160.02 118.745) (size 0.8) (drill 0.4) (layers F.Cu B.Cu) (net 29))
 (segment (start 160.29 118.475) (end 160.02 118.745) (width 0.25) (layer F.Cu) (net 29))
 (segment (start 160.29 116.585) (end 160.29 118.475) (width 0.25) (layer F.Cu) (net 29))
 (via (at 162.56 118.745) (size 0.8) (drill 0.4) (layers F.Cu B.Cu) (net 30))
 (segment (start 162.56 116.855) (end 162.29 116.585) (width 0.25) (layer F.Cu) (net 30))
 (segment (start 162.56 118.745) (end 162.56 116.855) (width 0.25) (layer F.Cu) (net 30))
 (via (at 162.56 79.375) (size 0.8) (drill 0.4) (layers F.Cu B.Cu) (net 30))
 (segment (start 153.915 79.375) (end 162.56 79.375) (width 0.25) (layer F.Cu) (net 30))
 (segment (start 162.56 117.475) (end 162.56 118.745) (width 0.25) (layer B.Cu) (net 30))
 (segment (start 162.56 79.375) (end 162.56 117.475) (width 0.25) (layer B.Cu) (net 30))
 (via (at 156.21 78.105) (size 0.8) (drill 0.4) (layers F.Cu B.Cu) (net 31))
 (segment (start 153.915 78.105) (end 156.21 78.105) (width 0.25) (layer F.Cu) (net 31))
 (via (at 156.21 118.745) (size 0.8) (drill 0.4) (layers F.Cu B.Cu) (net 31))
 (segment (start 156.21 78.105) (end 156.21 118.745) (width 0.25) (layer B.Cu) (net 31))
 (segment (start 156.21 116.665) (end 156.29 116.585) (width 0.25) (layer F.Cu) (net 31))
 (segment (start 156.21 118.745) (end 156.21 116.665) (width 0.25) (layer F.Cu) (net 31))
 (via (at 164.465 70.485) (size 0.8) (drill 0.4) (layers F.Cu B.Cu) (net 37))
 (segment (start 155.165 70.485) (end 153.915 70.485) (width 0.25) (layer F.Cu) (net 37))
 (segment (start 164.465 70.485) (end 155.165 70.485) (width 0.25) (layer F.Cu) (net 37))
 (segment (start 164.465 70.485) (end 164.465 118.745) (width 0.25) (layer B.Cu) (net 37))
 (segment (start 164.465 118.745) (end 164.465 118.745) (width 0.25) (layer B.Cu) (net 37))
 (via (at 164.465 118.745) (size 0.8) (drill 0.4) (layers F.Cu B.Cu) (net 37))
 (segment (start 164.465 116.76) (end 164.29 116.585) (width 0.25) (layer F.Cu) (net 37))
 (segment (start 164.465 118.745) (end 164.465 116.76) (width 0.25) (layer F.Cu) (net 37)))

